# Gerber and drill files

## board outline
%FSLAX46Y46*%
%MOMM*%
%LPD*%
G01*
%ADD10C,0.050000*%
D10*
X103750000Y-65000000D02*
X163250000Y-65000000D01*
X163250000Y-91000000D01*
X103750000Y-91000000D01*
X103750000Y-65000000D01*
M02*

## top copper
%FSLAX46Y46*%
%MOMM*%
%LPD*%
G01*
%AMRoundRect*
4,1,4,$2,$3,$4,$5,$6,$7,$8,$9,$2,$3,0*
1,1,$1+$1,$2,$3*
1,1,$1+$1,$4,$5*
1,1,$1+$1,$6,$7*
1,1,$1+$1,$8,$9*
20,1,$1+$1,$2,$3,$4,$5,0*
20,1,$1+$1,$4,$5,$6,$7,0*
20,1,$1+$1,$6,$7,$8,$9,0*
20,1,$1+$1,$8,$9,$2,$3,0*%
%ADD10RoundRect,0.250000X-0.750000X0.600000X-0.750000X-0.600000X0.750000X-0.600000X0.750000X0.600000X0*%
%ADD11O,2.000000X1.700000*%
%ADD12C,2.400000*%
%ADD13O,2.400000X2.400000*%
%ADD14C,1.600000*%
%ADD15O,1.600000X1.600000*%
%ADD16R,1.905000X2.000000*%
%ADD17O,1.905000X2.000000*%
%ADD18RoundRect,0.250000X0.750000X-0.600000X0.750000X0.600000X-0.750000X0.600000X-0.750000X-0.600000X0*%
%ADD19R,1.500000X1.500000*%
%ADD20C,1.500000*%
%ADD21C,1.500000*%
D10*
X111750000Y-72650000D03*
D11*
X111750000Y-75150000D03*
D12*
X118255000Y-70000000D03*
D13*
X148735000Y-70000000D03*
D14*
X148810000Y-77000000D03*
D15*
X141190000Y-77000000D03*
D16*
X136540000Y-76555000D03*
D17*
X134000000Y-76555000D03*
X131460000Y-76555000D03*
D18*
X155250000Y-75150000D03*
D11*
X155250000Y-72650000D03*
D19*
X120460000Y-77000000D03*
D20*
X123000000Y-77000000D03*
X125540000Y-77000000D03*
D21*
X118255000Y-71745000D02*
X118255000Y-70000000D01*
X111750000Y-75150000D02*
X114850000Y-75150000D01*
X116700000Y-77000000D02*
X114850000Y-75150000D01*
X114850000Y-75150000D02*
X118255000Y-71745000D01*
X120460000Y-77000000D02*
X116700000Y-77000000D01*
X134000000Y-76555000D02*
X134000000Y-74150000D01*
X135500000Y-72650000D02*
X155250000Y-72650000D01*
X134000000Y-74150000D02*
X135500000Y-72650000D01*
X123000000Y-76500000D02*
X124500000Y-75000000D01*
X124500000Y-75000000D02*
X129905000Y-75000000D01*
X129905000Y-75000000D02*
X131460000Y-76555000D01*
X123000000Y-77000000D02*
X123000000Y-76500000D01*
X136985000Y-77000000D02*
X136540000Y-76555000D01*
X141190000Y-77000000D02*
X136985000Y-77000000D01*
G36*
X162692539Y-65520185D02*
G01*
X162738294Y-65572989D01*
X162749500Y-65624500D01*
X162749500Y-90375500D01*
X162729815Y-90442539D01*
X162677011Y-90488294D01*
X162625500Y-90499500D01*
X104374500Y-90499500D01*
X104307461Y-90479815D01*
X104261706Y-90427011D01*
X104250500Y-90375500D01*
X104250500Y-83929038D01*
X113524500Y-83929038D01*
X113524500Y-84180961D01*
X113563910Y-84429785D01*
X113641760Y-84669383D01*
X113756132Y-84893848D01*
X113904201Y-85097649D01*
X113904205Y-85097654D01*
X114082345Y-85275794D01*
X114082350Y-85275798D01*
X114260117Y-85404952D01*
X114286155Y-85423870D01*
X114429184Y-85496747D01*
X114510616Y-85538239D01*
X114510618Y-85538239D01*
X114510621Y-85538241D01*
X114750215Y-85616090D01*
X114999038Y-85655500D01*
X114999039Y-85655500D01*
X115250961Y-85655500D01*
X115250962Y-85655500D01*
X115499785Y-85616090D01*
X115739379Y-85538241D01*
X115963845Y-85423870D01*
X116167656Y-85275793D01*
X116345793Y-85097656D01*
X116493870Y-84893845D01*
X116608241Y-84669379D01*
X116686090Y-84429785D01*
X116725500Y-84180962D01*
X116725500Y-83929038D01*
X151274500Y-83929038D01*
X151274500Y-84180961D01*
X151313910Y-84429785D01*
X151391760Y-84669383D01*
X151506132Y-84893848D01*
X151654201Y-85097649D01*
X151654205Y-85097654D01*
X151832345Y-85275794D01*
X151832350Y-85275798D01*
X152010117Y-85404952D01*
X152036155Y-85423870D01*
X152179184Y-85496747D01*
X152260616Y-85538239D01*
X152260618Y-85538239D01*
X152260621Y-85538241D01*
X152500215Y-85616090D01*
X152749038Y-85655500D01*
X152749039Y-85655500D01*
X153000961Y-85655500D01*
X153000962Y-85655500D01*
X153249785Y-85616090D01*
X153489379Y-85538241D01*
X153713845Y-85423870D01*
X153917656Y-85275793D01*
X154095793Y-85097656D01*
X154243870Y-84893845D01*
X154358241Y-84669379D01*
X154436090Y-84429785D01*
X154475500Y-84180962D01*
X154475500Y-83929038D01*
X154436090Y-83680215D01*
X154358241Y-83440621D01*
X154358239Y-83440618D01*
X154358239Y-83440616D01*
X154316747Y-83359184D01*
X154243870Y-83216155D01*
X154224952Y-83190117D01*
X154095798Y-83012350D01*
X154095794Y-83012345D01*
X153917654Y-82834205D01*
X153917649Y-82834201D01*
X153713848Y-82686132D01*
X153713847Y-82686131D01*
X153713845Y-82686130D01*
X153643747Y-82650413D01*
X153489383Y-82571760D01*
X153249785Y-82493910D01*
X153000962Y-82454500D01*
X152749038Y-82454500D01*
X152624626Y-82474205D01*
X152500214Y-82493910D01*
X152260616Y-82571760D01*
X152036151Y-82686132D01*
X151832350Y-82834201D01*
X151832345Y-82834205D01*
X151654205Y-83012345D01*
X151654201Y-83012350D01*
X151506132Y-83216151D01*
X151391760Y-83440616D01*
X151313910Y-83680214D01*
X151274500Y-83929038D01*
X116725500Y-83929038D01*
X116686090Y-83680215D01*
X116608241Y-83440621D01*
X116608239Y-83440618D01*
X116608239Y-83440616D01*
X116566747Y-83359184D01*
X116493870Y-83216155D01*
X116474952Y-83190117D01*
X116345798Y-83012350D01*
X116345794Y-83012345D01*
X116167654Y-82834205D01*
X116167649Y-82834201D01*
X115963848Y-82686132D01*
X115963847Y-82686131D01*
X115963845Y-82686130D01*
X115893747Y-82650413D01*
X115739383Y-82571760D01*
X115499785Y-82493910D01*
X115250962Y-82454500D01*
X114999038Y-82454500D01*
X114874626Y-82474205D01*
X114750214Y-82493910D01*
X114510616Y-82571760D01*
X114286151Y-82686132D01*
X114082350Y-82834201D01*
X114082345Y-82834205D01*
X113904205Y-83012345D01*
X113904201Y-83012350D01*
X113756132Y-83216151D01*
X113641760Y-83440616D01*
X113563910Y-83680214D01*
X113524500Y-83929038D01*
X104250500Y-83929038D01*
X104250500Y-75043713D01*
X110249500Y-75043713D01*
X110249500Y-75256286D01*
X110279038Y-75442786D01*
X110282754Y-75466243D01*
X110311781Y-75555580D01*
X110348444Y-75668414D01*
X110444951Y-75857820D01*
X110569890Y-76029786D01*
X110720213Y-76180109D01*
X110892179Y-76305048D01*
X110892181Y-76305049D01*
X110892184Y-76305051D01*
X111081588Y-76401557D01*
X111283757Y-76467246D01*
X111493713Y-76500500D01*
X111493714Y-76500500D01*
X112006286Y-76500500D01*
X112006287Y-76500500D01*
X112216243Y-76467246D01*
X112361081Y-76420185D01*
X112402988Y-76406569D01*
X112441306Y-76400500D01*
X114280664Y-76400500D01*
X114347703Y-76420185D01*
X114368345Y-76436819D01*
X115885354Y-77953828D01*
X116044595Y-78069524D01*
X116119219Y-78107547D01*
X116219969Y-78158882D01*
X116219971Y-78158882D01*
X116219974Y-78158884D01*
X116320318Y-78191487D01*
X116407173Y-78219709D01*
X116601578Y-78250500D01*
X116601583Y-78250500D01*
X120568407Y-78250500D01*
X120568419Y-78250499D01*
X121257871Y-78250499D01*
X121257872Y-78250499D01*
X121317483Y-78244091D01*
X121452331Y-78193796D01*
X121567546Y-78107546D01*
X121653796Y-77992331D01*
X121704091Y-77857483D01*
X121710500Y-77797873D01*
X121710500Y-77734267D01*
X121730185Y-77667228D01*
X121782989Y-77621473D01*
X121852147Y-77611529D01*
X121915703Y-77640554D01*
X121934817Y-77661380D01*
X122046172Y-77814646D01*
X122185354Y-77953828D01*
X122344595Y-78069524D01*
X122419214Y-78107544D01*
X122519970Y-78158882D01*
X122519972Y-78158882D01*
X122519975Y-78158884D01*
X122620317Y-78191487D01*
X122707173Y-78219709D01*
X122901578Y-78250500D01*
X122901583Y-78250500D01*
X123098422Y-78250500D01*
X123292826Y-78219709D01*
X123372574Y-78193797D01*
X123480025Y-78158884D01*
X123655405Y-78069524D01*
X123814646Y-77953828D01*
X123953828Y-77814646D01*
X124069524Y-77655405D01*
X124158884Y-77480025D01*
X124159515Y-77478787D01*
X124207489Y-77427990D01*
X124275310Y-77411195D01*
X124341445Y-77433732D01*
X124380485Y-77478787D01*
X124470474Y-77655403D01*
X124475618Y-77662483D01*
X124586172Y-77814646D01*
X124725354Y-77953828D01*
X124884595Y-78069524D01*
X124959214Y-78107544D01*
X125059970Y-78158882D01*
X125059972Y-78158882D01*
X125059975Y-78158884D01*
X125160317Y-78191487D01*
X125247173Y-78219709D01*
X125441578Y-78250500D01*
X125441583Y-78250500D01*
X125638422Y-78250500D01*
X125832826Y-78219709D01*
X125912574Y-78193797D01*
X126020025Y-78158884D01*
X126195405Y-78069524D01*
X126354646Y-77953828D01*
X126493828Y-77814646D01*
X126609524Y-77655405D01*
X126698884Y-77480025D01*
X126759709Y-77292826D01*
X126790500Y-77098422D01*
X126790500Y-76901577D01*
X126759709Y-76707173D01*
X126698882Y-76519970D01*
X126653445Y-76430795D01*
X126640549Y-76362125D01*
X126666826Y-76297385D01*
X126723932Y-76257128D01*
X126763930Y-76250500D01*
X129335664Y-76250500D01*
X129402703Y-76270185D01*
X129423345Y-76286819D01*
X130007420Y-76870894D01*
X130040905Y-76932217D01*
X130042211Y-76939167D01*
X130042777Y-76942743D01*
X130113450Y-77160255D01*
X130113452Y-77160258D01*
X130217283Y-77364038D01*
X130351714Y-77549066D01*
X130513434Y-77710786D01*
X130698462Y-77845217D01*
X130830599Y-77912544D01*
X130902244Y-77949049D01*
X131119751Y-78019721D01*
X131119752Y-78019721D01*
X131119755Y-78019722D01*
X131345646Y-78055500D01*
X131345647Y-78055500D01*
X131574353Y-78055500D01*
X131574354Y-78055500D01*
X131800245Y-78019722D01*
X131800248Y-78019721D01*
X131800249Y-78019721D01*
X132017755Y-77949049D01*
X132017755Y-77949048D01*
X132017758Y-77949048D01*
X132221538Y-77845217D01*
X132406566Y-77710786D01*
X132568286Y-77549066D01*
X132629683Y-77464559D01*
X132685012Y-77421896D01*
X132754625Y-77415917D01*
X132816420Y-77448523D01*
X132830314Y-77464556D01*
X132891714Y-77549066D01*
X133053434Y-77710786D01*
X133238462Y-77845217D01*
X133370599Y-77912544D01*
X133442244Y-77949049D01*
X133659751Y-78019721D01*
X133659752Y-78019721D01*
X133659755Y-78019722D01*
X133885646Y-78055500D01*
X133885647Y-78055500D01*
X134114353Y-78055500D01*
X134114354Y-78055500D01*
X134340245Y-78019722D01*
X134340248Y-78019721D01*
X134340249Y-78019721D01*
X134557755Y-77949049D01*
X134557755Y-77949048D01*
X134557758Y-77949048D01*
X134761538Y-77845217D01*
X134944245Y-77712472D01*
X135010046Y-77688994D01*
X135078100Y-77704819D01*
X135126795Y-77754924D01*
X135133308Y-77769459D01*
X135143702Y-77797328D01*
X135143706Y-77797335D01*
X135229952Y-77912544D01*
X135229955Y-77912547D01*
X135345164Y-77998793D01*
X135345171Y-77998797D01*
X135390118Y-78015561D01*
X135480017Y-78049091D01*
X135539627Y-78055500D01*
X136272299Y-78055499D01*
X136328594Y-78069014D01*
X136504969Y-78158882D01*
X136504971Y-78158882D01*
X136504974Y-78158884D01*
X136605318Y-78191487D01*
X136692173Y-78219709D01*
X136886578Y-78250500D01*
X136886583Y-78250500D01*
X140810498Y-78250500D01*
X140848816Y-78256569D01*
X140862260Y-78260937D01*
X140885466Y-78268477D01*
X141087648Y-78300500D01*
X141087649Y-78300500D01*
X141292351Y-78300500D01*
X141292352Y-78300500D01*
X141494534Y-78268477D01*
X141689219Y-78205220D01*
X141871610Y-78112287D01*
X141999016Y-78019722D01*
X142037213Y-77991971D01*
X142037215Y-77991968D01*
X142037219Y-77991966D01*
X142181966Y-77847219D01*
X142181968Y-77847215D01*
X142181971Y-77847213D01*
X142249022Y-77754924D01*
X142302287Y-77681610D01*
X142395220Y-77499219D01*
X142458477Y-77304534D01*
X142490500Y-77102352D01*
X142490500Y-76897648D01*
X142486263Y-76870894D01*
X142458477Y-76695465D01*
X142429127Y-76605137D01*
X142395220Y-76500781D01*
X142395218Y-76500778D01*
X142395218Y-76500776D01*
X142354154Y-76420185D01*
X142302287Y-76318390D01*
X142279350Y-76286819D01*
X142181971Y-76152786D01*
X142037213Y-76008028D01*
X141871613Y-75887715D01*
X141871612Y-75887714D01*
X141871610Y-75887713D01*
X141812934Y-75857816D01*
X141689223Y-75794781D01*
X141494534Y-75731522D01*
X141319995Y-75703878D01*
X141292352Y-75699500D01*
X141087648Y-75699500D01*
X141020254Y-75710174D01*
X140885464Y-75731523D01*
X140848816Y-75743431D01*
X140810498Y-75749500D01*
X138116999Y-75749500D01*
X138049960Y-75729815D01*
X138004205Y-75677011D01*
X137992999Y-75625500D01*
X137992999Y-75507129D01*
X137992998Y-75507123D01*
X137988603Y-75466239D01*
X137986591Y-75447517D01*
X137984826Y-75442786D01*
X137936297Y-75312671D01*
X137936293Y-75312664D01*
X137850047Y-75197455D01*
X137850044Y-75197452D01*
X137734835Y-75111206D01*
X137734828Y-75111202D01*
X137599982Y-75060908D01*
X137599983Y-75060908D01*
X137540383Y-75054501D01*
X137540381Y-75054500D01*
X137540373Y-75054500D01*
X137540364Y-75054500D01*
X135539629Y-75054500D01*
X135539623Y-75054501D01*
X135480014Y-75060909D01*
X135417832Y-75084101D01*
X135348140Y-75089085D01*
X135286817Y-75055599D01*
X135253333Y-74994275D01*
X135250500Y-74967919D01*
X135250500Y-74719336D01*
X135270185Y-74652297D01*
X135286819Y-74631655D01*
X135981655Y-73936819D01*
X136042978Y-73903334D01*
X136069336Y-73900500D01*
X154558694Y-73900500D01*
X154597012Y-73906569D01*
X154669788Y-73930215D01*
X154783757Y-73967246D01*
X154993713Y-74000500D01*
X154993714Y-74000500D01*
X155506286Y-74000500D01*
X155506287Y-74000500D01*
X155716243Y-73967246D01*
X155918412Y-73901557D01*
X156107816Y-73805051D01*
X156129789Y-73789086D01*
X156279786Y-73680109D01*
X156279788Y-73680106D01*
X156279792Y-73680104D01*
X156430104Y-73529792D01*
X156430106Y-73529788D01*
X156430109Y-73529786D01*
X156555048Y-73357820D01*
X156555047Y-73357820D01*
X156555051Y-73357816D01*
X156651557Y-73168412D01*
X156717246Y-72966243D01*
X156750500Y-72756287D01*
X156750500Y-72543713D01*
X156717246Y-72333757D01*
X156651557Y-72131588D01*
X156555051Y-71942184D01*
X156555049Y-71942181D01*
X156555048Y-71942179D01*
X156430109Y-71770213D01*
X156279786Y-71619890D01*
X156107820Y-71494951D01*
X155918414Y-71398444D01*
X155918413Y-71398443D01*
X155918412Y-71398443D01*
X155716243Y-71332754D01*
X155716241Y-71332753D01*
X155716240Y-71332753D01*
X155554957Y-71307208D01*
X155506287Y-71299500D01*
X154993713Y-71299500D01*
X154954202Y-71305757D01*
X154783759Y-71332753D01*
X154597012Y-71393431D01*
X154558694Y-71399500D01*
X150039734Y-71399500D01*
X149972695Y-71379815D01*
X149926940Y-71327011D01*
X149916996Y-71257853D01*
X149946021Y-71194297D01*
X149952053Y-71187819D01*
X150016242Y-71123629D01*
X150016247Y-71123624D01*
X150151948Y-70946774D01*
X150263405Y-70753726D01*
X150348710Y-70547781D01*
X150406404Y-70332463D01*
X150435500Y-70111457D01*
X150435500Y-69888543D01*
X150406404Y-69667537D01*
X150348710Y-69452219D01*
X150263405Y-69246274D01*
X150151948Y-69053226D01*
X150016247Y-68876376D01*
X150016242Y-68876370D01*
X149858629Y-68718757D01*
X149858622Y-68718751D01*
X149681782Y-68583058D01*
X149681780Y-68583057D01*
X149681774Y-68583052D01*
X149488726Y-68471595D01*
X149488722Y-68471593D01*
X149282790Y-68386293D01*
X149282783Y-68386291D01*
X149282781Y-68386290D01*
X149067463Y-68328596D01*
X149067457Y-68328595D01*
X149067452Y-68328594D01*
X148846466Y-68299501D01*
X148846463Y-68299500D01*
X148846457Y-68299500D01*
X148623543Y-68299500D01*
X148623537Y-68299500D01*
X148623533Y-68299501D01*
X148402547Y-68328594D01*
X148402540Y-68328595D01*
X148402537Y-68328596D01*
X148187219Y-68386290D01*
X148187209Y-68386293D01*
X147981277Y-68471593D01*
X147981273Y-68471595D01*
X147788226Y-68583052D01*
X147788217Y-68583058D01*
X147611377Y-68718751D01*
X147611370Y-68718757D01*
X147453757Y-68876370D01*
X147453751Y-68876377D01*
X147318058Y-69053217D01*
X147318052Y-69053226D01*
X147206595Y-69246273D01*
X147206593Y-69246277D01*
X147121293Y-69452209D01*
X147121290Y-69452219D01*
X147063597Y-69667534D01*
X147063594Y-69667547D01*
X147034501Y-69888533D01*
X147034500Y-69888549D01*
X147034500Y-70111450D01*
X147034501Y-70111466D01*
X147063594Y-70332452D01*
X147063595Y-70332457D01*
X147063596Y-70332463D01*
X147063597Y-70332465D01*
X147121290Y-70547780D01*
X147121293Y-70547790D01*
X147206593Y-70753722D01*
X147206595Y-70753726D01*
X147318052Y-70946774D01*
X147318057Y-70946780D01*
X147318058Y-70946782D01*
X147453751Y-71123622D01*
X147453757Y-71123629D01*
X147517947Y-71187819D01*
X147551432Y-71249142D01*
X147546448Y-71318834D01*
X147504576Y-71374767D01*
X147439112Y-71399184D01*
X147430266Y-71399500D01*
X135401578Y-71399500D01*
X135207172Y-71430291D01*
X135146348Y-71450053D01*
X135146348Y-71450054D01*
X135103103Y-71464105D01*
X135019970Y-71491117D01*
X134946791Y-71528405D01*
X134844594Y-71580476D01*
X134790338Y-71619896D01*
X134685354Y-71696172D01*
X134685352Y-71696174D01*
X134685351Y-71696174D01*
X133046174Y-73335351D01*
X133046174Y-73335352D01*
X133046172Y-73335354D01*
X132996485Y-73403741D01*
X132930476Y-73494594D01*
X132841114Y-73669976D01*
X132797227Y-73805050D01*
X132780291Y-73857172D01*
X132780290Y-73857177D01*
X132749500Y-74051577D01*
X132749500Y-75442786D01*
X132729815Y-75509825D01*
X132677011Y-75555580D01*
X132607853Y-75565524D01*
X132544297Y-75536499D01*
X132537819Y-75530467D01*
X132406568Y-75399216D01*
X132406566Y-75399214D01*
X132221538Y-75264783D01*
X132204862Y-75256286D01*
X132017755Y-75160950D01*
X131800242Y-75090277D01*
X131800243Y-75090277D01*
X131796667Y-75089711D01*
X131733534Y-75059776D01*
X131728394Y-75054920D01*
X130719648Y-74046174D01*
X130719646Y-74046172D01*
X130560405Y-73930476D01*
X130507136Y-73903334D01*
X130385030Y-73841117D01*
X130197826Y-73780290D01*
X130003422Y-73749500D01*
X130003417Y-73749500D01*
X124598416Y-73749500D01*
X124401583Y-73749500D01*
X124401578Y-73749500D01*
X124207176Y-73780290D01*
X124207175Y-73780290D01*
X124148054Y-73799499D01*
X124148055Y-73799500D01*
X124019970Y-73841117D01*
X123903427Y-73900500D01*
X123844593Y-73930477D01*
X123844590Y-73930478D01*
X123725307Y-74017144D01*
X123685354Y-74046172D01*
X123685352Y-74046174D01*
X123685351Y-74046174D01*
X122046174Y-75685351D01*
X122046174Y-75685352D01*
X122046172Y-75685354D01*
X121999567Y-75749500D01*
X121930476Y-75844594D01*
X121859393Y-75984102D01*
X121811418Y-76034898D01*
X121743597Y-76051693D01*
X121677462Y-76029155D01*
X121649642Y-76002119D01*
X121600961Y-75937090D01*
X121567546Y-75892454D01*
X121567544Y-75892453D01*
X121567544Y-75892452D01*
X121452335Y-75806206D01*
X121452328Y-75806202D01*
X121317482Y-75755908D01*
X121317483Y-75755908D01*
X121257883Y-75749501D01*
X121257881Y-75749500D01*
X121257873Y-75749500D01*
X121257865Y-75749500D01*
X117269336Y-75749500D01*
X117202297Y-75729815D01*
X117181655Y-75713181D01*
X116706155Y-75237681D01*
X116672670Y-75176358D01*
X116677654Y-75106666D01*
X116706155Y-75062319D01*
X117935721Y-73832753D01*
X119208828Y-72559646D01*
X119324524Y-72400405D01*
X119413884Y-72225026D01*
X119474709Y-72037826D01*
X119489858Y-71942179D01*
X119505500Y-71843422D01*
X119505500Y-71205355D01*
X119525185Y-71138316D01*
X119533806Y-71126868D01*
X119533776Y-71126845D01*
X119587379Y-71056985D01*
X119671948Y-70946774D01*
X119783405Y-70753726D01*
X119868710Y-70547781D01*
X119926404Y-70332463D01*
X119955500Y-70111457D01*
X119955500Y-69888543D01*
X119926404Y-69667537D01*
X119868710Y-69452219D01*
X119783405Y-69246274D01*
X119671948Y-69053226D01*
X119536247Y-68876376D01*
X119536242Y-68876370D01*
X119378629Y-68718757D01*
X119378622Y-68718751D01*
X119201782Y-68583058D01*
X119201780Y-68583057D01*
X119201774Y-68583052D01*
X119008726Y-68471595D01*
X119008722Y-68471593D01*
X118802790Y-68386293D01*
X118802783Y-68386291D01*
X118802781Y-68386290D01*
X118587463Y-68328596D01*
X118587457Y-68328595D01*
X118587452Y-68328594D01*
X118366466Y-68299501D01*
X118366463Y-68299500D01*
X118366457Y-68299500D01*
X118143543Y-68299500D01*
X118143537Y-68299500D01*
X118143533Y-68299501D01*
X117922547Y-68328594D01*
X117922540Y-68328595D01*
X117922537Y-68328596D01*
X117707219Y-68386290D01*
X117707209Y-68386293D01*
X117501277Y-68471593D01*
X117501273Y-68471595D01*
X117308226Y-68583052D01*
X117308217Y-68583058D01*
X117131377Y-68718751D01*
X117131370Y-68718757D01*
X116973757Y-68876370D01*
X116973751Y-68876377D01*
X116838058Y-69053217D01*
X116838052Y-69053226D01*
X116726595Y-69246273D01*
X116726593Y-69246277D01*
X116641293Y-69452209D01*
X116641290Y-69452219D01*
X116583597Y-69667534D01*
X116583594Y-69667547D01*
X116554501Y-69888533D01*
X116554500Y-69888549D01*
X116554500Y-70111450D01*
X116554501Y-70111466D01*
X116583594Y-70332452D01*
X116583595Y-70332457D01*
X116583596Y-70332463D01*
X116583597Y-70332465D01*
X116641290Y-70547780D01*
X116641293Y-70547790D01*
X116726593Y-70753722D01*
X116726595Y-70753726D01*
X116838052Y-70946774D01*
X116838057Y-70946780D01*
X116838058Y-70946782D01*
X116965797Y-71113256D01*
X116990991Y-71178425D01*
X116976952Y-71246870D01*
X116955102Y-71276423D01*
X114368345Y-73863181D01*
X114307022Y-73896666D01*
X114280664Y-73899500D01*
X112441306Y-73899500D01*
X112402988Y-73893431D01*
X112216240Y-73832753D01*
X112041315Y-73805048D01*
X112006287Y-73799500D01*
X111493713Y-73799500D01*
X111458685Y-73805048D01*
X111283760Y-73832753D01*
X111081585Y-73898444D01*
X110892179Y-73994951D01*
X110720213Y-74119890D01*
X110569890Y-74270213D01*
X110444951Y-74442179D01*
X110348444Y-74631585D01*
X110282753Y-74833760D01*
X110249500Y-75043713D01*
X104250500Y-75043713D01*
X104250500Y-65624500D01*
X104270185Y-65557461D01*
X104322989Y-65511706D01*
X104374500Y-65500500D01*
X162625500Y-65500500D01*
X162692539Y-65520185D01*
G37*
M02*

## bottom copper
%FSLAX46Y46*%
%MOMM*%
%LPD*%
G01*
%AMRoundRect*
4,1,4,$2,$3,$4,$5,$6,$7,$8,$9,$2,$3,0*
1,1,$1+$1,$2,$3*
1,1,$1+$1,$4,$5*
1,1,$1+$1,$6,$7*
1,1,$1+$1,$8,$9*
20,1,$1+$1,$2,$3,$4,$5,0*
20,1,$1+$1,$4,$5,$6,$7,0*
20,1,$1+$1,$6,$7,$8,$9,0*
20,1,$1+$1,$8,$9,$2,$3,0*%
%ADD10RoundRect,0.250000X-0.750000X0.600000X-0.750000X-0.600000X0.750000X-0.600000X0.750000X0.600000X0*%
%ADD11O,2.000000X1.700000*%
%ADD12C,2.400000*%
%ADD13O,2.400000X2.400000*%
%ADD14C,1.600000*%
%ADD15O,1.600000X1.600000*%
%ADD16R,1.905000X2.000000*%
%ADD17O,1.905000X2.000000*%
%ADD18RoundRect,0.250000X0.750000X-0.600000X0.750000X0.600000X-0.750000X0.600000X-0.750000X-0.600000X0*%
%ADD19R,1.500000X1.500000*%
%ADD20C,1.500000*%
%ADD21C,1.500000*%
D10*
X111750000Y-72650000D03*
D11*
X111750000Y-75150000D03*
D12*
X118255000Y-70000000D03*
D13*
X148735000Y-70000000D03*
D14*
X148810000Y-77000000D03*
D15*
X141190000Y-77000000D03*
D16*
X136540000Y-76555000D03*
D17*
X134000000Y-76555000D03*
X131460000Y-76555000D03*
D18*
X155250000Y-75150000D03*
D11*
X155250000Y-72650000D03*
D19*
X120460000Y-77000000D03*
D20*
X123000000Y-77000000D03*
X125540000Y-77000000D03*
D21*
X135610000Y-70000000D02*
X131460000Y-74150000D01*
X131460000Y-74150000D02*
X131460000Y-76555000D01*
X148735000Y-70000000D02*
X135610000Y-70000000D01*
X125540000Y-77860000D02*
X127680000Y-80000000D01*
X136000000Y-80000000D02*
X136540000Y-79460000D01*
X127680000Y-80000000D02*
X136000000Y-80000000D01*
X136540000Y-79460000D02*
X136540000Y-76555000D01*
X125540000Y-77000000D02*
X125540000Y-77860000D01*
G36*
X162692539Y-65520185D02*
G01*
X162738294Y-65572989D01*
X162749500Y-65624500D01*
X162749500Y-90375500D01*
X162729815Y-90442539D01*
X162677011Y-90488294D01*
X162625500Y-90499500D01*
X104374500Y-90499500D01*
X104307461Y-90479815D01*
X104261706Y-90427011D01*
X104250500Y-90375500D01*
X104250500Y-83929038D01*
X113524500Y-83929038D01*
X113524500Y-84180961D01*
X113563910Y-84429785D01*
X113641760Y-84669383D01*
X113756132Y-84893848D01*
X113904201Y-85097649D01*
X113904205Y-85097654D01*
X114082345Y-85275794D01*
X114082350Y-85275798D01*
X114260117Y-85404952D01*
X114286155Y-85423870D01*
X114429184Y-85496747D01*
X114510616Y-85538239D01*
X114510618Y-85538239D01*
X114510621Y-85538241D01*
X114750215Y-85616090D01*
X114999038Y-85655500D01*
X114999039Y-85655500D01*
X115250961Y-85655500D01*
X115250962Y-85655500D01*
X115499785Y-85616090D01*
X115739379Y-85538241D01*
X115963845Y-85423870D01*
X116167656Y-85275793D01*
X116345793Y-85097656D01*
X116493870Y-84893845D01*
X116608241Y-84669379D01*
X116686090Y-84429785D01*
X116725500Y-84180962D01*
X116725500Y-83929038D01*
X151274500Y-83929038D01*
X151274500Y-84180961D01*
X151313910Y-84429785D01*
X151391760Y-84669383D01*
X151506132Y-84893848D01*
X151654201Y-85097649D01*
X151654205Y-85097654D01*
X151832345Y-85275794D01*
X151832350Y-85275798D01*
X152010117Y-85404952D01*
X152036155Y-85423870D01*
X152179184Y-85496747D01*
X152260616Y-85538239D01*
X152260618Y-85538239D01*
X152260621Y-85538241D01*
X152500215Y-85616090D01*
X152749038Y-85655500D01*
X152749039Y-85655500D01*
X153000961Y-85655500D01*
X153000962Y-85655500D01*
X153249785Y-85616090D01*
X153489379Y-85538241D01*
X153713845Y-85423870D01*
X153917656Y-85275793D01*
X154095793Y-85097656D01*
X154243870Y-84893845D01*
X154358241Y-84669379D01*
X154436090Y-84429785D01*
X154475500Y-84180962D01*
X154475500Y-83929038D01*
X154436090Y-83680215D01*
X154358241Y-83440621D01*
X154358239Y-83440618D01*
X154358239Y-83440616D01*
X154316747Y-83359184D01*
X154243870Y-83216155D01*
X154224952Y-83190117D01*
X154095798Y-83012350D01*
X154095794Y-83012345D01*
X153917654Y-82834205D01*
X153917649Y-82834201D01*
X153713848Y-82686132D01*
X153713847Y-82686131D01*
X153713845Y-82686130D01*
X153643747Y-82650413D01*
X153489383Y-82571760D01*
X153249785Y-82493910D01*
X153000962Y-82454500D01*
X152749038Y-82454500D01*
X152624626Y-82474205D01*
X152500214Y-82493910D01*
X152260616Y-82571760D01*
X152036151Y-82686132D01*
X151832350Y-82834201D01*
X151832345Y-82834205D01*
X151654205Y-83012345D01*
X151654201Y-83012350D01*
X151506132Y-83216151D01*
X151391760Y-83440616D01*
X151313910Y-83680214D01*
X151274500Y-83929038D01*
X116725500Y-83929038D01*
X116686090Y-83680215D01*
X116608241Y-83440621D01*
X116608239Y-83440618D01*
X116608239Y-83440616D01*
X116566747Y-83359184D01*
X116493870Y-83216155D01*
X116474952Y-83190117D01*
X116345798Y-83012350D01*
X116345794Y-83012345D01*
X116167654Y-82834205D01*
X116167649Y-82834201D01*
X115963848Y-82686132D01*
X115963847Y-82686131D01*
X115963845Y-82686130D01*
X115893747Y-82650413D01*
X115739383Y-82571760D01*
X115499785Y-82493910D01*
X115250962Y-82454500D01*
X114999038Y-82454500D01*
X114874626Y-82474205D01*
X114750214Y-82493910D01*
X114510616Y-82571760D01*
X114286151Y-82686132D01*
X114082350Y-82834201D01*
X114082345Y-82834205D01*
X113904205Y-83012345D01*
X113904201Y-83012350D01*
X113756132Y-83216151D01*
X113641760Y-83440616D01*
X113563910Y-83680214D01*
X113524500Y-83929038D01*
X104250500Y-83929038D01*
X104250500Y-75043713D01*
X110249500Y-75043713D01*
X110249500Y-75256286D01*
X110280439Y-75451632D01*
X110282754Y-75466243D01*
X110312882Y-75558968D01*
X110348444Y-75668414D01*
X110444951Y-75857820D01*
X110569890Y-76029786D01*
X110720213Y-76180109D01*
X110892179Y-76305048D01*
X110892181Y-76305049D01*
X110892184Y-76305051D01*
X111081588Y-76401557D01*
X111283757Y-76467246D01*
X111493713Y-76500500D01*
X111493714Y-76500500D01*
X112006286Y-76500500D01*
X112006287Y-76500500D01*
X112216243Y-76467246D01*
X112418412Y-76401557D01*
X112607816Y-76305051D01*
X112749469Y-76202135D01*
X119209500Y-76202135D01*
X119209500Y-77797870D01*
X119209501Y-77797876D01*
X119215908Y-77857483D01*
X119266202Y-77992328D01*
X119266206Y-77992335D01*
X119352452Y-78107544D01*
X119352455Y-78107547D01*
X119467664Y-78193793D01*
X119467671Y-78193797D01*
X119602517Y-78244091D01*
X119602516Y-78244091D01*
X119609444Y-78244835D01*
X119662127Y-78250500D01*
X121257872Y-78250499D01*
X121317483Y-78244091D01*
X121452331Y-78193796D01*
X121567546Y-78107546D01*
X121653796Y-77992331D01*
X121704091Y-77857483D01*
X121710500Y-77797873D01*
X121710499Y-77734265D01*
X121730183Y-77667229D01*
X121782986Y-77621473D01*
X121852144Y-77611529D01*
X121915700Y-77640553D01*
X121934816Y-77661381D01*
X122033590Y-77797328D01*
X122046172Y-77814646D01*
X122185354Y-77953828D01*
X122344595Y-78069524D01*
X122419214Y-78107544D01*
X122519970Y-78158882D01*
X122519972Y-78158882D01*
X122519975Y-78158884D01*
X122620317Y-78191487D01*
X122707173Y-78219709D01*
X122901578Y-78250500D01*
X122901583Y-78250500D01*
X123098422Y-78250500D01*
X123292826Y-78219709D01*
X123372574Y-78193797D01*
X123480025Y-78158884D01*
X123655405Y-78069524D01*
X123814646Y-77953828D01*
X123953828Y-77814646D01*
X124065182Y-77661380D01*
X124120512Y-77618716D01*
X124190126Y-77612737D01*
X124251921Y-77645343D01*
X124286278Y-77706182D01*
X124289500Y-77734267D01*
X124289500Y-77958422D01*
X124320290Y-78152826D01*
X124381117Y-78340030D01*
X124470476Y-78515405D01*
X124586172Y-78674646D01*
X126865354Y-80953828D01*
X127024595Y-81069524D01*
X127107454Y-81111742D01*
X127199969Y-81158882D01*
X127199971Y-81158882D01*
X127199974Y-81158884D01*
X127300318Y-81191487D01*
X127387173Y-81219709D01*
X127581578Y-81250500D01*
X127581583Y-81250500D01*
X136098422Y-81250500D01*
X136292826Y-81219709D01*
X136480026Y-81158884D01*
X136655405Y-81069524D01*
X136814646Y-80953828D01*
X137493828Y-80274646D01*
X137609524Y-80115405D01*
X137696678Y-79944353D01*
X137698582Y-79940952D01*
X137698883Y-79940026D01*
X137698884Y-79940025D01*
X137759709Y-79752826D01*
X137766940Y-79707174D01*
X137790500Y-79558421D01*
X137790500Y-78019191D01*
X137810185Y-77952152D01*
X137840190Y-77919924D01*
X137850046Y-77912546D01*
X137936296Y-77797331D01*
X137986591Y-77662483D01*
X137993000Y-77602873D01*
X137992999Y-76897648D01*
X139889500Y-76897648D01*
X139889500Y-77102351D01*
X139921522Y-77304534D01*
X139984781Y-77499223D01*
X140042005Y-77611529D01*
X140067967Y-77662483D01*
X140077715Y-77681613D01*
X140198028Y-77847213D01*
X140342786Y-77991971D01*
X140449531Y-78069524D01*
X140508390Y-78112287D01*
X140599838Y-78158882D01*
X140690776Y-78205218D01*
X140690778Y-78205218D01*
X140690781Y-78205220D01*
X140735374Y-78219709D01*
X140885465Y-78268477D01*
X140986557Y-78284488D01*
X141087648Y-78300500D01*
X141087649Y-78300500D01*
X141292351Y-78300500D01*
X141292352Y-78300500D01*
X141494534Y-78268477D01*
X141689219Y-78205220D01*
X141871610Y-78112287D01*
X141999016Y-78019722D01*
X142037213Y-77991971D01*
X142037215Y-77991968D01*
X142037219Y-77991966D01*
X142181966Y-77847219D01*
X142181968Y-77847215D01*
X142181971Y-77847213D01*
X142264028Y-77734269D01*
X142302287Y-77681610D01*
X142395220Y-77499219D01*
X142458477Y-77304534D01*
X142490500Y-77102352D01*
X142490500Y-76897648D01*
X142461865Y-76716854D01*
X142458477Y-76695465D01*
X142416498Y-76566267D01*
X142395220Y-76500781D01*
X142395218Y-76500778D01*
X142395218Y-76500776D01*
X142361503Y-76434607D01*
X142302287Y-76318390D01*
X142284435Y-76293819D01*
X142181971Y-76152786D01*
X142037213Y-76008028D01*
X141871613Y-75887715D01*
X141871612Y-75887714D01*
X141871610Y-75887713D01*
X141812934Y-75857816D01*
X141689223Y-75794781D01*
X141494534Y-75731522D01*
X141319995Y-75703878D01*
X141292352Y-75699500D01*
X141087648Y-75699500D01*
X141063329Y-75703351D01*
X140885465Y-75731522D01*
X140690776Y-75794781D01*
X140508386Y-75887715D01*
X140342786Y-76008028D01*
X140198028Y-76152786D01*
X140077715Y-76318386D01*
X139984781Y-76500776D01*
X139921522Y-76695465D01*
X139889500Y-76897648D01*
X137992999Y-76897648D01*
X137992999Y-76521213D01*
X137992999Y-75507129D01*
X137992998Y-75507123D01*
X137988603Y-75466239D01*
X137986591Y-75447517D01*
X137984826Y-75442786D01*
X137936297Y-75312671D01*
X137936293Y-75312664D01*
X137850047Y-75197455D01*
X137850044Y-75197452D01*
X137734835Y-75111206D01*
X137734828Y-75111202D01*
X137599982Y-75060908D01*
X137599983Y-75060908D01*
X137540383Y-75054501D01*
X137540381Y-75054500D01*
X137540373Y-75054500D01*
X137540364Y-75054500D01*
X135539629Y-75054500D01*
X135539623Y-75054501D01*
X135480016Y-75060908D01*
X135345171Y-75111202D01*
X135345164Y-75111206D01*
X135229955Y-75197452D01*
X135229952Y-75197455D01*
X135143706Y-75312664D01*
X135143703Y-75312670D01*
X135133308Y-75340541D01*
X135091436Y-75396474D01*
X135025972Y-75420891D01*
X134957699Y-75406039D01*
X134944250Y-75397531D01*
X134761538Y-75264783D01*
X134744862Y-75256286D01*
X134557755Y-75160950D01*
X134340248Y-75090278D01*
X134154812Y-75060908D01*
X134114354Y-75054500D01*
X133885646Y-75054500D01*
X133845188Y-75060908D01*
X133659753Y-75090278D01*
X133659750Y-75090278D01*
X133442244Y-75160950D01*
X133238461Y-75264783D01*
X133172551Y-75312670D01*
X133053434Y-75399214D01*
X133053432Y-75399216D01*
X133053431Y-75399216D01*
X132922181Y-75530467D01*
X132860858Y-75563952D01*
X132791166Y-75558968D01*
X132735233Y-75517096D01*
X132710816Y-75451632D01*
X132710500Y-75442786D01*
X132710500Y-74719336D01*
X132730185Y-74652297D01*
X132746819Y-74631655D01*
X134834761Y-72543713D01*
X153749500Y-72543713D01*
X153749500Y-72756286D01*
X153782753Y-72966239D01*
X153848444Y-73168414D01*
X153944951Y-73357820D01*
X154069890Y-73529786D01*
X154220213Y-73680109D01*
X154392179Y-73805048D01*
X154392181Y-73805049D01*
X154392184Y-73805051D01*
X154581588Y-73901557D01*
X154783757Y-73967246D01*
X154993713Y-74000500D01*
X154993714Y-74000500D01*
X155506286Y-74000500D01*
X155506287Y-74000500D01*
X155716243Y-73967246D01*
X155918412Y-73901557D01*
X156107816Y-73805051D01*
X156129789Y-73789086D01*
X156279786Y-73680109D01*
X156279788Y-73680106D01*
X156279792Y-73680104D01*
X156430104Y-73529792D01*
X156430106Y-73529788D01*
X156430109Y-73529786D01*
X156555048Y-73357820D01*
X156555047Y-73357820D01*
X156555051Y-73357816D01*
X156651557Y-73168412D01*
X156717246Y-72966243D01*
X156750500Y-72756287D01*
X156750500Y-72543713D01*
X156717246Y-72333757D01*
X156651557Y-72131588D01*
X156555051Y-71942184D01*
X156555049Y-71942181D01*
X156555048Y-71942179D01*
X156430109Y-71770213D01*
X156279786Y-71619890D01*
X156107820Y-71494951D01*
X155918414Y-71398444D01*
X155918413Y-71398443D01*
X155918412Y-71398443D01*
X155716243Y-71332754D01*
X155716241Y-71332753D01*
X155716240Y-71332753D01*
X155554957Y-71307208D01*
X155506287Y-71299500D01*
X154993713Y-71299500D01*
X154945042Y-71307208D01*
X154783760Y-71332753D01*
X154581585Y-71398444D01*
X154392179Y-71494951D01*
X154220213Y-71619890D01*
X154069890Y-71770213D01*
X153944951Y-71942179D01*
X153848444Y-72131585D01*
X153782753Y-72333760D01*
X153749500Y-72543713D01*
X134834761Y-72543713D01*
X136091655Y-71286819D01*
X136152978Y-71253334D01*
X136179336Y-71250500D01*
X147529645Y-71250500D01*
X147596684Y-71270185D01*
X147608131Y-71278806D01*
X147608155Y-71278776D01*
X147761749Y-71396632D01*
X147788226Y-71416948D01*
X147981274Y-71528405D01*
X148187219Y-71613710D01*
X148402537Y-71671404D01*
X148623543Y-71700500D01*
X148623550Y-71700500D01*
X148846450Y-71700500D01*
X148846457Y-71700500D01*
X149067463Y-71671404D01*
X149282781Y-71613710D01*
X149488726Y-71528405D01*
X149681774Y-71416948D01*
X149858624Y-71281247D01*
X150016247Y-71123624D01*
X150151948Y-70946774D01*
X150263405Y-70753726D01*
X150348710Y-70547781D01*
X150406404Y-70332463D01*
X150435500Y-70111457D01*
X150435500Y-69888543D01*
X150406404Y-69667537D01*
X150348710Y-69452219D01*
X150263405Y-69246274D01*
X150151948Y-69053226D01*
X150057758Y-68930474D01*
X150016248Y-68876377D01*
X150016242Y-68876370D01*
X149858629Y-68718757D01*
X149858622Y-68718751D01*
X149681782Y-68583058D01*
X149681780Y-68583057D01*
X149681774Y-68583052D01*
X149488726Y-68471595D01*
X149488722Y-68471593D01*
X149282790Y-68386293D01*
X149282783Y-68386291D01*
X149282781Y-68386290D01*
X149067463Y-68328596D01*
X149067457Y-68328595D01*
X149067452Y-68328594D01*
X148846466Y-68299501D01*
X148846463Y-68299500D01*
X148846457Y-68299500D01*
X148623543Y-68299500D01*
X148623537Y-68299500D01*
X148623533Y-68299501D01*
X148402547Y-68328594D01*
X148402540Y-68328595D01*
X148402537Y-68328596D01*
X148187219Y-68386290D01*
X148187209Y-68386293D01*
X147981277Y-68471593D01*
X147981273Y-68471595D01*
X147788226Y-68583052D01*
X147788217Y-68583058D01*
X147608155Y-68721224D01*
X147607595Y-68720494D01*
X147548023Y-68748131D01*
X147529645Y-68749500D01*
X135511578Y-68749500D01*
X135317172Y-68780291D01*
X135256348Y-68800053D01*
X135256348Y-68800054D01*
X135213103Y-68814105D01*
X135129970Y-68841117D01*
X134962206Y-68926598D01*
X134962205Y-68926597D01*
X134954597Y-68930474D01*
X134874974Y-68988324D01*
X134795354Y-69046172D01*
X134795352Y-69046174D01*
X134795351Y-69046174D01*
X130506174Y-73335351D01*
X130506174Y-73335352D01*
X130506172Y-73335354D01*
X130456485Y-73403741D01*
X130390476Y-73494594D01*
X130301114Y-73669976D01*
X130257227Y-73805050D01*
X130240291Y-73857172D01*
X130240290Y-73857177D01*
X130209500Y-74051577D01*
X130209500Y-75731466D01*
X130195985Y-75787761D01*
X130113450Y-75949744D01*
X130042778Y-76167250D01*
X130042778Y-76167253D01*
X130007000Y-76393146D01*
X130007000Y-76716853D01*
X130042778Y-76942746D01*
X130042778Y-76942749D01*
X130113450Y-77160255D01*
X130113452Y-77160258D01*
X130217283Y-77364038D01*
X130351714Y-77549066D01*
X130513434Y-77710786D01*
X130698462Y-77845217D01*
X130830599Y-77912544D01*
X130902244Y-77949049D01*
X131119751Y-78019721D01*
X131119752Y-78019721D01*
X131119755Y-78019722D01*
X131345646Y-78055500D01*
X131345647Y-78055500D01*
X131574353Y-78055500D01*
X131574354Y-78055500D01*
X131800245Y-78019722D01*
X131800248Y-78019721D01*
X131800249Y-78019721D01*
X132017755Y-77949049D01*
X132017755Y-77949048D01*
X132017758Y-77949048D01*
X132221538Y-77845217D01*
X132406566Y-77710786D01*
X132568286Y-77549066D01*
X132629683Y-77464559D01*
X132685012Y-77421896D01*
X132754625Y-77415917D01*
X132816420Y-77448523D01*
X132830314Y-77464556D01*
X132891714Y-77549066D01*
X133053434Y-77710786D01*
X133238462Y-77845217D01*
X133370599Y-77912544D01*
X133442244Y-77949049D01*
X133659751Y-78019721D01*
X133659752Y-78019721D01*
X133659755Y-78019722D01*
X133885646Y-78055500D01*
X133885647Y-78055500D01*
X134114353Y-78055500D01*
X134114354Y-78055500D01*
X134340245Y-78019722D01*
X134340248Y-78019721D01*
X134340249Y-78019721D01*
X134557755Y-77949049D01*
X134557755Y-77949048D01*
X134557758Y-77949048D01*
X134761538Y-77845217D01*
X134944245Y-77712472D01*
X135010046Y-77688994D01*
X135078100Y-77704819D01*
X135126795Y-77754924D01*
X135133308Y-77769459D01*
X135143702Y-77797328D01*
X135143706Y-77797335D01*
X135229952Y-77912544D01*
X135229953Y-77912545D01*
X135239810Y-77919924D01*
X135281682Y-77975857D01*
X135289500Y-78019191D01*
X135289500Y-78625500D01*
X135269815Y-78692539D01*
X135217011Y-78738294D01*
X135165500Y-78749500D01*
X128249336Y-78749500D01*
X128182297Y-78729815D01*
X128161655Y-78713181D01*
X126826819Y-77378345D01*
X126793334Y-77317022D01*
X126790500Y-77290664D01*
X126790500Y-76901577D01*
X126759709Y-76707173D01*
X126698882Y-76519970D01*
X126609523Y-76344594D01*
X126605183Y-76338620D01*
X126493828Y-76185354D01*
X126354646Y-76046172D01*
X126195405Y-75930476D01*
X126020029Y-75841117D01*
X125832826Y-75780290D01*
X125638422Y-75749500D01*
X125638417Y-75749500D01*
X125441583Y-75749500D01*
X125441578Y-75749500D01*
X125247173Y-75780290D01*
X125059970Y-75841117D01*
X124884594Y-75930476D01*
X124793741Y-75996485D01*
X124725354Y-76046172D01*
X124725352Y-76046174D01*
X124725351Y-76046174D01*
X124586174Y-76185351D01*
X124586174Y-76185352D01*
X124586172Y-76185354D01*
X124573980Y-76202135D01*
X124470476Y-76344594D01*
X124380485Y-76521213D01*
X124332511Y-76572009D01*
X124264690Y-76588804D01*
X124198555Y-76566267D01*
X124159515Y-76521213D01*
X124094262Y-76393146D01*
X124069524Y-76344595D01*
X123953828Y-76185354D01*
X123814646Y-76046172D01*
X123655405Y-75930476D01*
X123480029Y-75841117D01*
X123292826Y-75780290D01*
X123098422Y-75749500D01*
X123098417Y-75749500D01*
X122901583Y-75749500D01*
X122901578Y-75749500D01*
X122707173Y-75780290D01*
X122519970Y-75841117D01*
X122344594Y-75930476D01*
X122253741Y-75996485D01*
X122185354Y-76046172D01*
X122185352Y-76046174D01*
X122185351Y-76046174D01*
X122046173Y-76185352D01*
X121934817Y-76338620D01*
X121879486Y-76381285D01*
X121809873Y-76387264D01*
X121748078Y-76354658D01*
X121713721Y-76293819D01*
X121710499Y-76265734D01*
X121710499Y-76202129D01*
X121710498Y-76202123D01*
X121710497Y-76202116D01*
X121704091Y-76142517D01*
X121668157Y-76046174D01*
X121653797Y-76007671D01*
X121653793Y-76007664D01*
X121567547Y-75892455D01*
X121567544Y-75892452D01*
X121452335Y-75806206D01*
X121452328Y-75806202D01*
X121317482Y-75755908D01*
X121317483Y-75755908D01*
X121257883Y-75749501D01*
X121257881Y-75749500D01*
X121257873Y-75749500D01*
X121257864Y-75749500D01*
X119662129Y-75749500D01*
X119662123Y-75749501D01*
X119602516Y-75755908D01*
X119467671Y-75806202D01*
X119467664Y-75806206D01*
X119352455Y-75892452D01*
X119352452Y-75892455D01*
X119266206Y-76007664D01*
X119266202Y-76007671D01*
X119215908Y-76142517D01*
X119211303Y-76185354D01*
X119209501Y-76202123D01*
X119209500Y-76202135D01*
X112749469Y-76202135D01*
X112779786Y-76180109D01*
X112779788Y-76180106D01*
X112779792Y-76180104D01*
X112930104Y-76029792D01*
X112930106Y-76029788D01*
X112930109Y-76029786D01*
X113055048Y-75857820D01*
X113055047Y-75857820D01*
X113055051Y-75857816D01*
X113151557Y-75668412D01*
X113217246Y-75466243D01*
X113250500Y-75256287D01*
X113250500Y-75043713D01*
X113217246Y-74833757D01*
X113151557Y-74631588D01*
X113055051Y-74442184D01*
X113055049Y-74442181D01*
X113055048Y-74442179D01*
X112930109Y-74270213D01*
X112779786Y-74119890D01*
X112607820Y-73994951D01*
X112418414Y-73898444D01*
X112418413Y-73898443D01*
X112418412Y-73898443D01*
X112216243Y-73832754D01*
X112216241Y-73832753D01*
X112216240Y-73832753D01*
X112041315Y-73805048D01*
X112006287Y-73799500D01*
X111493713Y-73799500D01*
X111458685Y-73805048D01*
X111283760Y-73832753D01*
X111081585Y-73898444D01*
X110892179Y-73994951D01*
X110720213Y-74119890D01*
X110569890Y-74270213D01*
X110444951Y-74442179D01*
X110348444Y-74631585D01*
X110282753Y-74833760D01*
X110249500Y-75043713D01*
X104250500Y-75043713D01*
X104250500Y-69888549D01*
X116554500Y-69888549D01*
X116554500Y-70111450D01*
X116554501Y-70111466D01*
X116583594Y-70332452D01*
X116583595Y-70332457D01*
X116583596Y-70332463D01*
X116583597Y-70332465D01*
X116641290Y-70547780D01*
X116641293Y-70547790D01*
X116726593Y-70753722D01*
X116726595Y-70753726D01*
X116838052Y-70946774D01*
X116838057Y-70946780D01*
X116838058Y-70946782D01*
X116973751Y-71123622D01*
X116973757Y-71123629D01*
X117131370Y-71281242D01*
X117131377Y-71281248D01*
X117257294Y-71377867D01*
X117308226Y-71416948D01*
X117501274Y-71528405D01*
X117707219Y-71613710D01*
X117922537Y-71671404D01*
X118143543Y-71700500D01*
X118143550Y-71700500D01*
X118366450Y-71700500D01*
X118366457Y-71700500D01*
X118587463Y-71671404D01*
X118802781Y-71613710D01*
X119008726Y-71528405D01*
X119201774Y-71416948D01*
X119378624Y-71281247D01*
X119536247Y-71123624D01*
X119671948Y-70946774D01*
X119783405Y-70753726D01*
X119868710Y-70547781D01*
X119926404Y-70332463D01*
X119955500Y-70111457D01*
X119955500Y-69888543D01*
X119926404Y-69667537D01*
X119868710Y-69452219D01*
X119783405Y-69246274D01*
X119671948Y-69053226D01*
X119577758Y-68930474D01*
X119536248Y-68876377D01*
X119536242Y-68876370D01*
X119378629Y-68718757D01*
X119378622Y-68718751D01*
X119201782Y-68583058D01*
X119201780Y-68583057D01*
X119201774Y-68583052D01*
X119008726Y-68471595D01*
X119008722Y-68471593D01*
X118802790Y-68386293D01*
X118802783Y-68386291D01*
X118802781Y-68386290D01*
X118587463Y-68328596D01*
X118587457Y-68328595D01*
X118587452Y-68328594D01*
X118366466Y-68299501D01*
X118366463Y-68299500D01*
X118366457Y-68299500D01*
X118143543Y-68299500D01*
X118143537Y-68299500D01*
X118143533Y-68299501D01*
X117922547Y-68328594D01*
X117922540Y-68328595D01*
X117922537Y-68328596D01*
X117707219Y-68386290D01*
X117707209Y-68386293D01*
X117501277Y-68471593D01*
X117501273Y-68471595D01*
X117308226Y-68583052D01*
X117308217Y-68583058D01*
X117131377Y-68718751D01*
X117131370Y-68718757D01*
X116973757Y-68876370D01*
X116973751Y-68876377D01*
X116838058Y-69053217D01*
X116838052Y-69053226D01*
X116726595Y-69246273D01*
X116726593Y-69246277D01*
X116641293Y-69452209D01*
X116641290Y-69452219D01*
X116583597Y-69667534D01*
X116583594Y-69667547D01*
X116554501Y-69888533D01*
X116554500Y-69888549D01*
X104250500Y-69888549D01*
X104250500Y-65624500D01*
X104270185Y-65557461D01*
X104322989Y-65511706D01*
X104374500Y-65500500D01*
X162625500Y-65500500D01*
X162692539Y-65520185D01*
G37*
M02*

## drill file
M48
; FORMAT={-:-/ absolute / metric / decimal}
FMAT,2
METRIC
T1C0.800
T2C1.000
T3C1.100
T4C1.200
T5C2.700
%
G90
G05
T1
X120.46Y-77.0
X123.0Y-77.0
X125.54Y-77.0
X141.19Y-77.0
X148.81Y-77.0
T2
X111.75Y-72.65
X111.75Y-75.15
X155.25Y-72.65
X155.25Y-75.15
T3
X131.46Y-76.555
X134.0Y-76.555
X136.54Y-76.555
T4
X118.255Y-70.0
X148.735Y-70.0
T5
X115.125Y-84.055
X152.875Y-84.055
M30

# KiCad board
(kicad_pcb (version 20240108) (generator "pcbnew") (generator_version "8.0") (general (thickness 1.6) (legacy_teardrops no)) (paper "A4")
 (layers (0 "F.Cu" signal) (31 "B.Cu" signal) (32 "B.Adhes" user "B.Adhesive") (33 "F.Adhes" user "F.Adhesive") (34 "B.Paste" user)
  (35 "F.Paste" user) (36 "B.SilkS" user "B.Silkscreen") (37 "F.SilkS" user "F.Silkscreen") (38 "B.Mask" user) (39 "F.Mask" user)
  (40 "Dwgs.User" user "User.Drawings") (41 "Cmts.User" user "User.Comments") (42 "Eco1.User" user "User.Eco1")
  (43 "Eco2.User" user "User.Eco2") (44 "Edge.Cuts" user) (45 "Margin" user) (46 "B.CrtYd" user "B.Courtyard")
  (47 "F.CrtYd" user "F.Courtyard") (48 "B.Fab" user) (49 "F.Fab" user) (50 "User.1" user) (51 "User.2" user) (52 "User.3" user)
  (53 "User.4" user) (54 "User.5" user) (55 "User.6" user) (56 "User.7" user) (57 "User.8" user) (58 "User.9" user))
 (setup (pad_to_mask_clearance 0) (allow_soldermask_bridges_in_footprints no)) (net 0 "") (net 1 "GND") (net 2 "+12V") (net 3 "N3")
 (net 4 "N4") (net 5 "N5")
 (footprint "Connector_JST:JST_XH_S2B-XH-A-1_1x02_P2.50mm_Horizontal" (layer "F.Cu") (at 111.75 72.65 -90)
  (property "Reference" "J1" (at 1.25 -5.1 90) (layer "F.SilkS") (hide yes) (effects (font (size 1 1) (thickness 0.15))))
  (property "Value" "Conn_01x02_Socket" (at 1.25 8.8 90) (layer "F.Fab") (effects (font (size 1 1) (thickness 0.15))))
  (pad "1" thru_hole roundrect (at 0 0 270) (size 1.7 2) (drill 1) (layers "*.Cu" "*.Mask") (remove_unused_layers no)
   (roundrect_rratio 0.147059) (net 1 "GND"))
  (pad "2" thru_hole oval (at 2.5 0 270) (size 1.7 2) (drill 1) (layers "*.Cu" "*.Mask") (remove_unused_layers no) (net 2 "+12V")))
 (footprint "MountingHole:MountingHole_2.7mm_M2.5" (layer "F.Cu") (at 152.875 84.055)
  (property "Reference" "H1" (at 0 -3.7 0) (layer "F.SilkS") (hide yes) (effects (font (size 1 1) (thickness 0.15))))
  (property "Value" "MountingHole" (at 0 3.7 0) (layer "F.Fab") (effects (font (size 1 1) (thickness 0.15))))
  (pad "" np_thru_hole circle (at 0 0) (size 2.7 2.7) (drill 2.7) (layers "*.Cu" "*.Mask")))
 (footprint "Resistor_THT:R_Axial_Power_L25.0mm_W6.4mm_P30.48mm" (layer "F.Cu") (at 118.255 70)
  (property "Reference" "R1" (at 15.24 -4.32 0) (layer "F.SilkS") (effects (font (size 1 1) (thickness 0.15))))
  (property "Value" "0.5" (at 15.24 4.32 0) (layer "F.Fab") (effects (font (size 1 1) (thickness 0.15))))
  (pad "1" thru_hole circle (at 0 0) (size 2.4 2.4) (drill 1.2) (layers "*.Cu" "*.Mask") (remove_unused_layers no) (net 2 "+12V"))
  (pad "2" thru_hole oval (at 30.48 0) (size 2.4 2.4) (drill 1.2) (layers "*.Cu" "*.Mask") (remove_unused_layers no) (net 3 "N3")))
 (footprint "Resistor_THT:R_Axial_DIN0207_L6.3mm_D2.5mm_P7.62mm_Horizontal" (layer "F.Cu") (at 148.81 77 180)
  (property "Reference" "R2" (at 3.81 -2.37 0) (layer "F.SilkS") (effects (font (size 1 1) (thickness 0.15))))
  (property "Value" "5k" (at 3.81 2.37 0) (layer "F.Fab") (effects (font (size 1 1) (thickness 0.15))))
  (pad "1" thru_hole circle (at 0 0 180) (size 1.6 1.6) (drill 0.8) (layers "*.Cu" "*.Mask") (remove_unused_layers no) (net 1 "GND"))
  (pad "2" thru_hole oval (at 7.62 0 180) (size 1.6 1.6) (drill 0.8) (layers "*.Cu" "*.Mask") (remove_unused_layers no) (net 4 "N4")))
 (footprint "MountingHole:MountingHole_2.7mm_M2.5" (layer "F.Cu") (at 115.125 84.055)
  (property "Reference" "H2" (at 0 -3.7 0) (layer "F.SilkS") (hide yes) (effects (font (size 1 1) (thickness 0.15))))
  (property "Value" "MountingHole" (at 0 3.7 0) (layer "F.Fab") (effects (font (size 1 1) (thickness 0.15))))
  (pad "" np_thru_hole circle (at 0 0) (size 2.7 2.7) (drill 2.7) (layers "*.Cu" "*.Mask")))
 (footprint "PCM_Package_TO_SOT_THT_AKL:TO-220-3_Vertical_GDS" (layer "F.Cu") (at 136.54 76.555 180)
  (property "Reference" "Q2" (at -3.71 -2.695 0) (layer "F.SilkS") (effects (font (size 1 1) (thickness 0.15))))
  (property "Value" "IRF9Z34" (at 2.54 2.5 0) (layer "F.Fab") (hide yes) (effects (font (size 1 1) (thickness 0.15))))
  (pad "1" thru_hole rect (at 0 0 180) (size 1.905 2) (drill 1.1) (layers "*.Cu" "*.Mask") (remove_unused_layers no) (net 4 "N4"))
  (pad "2" thru_hole oval (at 2.54 0 180) (size 1.905 2) (drill 1.1) (layers "*.Cu" "*.Mask") (remove_unused_layers no) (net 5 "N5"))
  (pad "3" thru_hole oval (at 5.08 0 180) (size 1.905 2) (drill 1.1) (layers "*.Cu" "*.Mask") (remove_unused_layers no) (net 3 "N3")))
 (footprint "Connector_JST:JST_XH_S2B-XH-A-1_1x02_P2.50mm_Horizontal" (layer "F.Cu") (at 155.25 75.15 90)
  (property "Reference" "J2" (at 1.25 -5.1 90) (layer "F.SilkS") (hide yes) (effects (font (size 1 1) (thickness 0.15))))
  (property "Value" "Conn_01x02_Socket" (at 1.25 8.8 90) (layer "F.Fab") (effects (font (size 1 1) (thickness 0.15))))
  (pad "1" thru_hole roundrect (at 0 0 90) (size 1.7 2) (drill 1) (layers "*.Cu" "*.Mask") (remove_unused_layers no)
   (roundrect_rratio 0.147059) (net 1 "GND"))
  (pad "2" thru_hole oval (at 2.5 0 90) (size 1.7 2) (drill 1) (layers "*.Cu" "*.Mask") (remove_unused_layers no) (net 5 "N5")))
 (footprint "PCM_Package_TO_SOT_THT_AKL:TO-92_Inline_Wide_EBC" (layer "F.Cu") (at 120.46 77)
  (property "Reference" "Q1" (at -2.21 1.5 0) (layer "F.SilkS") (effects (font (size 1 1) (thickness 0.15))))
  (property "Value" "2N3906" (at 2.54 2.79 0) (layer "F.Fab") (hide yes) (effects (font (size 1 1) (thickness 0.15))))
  (pad "1" thru_hole rect (at 0 0 90) (size 1.5 1.5) (drill 0.8) (layers "*.Cu" "*.Mask") (remove_unused_layers no) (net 2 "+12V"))
  (pad "2" thru_hole circle (at 2.54 0 90) (size 1.5 1.5) (drill 0.8) (layers "*.Cu" "*.Mask") (remove_unused_layers no) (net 3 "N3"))
  (pad "3" thru_hole circle (at 5.08 0 90) (size 1.5 1.5) (drill 0.8) (layers "*.Cu" "*.Mask") (remove_unused_layers no) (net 4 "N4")))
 (gr_rect (start 103.75 65) (end 163.25 91) (stroke (width 0.05) (type default)) (fill none) (layer "Edge.Cuts"))
 (segment (start 118.255 71.745) (end 118.255 70) (width 1.5) (layer "F.Cu") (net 2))
 (segment (start 111.75 75.15) (end 114.85 75.15) (width 1.5) (layer "F.Cu") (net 2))
 (segment (start 116.7 77) (end 114.85 75.15) (width 1.5) (layer "F.Cu") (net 2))
 (segment (start 114.85 75.15) (end 118.255 71.745) (width 1.5) (layer "F.Cu") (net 2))
 (segment (start 120.46 77) (end 116.7 77) (width 1.5) (layer "F.Cu") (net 2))
 (segment (start 134 76.555) (end 134 74.15) (width 1.5) (layer "F.Cu") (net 5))
 (segment (start 135.5 72.65) (end 155.25 72.65) (width 1.5) (layer "F.Cu") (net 5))
 (segment (start 134 74.15) (end 135.5 72.65) (width 1.5) (layer "F.Cu") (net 5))
 (segment (start 123 76.5) (end 124.5 75) (width 1.5) (layer "F.Cu") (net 3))
 (segment (start 124.5 75) (end 129.905 75) (width 1.5) (layer "F.Cu") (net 3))
 (segment (start 129.905 75) (end 131.46 76.555) (width 1.5) (layer "F.Cu") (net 3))
 (segment (start 123 77) (end 123 76.5) (width 1.5) (layer "F.Cu") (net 3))
 (segment (start 135.61 70) (end 131.46 74.15) (width 1.5) (layer "B.Cu") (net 3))
 (segment (start 131.46 74.15) (end 131.46 76.555) (width 1.5) (layer "B.Cu") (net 3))
 (segment (start 148.735 70) (end 135.61 70) (width 1.5) (layer "B.Cu") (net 3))
 (segment (start 136.985 77) (end 136.54 76.555) (width 1.5) (layer "F.Cu") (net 4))
 (segment (start 141.19 77) (end 136.985 77) (width 1.5) (layer "F.Cu") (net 4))
 (segment (start 125.54 77.86) (end 127.68 80) (width 1.5) (layer "B.Cu") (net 4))
 (segment (start 136 80) (end 136.54 79.46) (width 1.5) (layer "B.Cu") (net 4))
 (segment (start 127.68 80) (end 136 80) (width 1.5) (layer "B.Cu") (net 4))
 (segment (start 136.54 79.46) (end 136.54 76.555) (width 1.5) (layer "B.Cu") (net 4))
 (segment (start 125.54 77) (end 125.54 77.86) (width 1.5) (layer "B.Cu") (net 4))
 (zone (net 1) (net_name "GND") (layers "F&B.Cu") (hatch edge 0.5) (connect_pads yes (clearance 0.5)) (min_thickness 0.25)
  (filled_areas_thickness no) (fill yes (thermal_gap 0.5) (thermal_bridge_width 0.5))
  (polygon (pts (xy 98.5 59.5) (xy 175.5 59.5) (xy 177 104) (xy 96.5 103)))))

